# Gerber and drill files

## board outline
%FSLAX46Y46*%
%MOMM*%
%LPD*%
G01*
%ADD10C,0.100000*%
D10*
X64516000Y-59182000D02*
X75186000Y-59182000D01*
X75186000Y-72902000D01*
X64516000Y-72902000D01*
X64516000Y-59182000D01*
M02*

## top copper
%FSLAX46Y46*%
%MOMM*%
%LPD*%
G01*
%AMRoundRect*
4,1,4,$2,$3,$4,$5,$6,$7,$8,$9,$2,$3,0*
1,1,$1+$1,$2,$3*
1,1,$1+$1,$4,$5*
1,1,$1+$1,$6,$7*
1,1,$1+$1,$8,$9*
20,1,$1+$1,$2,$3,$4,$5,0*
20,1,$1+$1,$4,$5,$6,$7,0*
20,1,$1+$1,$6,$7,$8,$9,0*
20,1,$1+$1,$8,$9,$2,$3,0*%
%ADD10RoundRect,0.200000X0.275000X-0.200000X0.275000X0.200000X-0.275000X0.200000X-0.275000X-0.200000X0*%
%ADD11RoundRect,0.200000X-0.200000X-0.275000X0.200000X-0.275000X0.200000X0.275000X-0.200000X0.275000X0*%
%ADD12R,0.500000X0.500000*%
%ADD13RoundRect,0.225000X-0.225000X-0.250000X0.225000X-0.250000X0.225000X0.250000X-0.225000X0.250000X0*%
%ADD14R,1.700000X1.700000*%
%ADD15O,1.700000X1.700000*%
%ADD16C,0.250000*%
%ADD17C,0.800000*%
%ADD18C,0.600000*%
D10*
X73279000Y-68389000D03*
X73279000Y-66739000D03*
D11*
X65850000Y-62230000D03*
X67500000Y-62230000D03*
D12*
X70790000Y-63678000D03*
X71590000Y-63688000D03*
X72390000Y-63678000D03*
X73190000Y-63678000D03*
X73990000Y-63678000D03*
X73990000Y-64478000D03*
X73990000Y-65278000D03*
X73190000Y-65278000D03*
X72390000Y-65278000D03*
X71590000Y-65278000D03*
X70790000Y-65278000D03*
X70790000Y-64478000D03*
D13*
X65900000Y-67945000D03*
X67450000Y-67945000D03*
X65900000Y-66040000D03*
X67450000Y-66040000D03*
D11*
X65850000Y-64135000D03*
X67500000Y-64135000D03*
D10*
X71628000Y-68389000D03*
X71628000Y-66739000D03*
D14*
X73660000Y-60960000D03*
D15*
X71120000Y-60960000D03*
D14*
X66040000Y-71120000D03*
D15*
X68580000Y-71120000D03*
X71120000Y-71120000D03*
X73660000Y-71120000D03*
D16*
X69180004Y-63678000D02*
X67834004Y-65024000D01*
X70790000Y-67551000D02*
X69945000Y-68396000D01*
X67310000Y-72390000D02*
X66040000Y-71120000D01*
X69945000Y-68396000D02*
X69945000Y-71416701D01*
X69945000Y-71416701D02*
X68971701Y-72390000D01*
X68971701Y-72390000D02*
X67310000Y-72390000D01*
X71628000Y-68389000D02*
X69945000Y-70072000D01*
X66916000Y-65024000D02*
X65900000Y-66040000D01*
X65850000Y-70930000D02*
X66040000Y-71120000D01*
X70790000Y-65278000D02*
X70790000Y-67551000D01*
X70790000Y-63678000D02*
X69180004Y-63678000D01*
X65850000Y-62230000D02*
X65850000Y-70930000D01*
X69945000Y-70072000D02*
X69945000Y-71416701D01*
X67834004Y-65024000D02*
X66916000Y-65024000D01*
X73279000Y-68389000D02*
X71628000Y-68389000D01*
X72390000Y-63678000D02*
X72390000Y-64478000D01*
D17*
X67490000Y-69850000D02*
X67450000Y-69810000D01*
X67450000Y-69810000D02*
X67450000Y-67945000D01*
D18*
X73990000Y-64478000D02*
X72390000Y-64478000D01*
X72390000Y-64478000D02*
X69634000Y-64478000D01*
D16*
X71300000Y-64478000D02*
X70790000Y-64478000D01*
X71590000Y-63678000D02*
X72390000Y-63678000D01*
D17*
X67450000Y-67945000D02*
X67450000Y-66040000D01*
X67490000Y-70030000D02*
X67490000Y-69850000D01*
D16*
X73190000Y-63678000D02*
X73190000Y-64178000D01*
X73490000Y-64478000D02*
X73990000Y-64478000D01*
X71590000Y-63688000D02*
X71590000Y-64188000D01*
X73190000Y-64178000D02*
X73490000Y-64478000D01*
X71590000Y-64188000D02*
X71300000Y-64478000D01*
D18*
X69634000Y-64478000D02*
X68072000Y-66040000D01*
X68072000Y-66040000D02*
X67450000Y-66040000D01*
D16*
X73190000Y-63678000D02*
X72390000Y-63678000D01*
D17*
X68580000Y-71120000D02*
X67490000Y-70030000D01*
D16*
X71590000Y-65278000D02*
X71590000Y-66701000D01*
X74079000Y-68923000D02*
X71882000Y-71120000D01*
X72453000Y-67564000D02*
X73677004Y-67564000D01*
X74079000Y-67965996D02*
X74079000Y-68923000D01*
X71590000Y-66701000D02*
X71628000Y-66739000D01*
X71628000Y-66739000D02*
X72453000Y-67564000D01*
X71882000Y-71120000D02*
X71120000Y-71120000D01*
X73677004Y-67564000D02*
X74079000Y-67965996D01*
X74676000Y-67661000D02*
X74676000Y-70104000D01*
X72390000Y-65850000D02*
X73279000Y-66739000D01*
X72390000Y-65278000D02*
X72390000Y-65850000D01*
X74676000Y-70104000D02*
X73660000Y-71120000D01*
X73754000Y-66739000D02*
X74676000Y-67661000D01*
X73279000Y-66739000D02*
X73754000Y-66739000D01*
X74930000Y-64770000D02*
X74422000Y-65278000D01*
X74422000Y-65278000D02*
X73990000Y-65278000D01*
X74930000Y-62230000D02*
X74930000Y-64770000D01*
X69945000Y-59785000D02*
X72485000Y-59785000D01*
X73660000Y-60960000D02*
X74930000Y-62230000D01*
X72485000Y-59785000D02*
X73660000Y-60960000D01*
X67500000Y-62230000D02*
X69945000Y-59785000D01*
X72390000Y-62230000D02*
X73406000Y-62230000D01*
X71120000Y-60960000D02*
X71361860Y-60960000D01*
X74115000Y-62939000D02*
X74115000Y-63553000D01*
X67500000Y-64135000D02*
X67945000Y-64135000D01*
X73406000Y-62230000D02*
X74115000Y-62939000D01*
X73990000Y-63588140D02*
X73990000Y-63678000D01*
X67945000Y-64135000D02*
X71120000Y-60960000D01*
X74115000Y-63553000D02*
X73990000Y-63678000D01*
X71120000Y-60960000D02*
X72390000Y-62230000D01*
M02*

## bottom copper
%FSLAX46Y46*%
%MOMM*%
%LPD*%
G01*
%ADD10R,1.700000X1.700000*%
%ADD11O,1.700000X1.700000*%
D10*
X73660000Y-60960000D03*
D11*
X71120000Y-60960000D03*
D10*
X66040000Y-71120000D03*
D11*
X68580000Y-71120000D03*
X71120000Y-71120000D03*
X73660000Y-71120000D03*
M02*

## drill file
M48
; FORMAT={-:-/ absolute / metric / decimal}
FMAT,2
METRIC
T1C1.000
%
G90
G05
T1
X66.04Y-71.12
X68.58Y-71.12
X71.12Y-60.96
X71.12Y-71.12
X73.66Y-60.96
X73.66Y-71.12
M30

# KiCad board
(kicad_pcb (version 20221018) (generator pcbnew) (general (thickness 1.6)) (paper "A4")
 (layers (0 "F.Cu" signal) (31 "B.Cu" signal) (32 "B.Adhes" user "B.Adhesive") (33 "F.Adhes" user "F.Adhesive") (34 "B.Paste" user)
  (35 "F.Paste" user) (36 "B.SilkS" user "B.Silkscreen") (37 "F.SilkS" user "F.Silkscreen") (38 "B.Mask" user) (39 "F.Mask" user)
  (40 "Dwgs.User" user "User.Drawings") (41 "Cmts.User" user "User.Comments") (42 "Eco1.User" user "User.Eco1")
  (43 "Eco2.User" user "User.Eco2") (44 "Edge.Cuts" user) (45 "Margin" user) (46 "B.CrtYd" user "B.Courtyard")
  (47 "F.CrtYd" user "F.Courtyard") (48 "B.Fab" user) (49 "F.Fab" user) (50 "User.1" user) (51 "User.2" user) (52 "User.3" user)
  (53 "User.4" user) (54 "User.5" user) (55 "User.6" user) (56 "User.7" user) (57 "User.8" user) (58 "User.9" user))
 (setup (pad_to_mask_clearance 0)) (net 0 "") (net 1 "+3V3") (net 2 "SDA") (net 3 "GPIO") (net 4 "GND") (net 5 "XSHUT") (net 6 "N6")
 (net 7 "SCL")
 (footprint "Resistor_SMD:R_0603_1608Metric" (layer "F.Cu") (at 73.279 67.564 90)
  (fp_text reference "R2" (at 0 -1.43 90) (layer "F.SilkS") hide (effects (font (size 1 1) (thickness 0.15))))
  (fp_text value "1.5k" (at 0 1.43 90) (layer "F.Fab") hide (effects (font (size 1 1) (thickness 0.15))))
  (pad "1" smd roundrect (at -0.825 0 90) (size 0.8 0.95) (layers "F.Cu" "F.Paste" "F.Mask") (roundrect_rratio 0.25) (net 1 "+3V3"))
  (pad "2" smd roundrect (at 0.825 0 90) (size 0.8 0.95) (layers "F.Cu" "F.Paste" "F.Mask") (roundrect_rratio 0.25) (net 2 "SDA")))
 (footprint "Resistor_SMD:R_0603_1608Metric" (layer "F.Cu") (at 66.675 62.23)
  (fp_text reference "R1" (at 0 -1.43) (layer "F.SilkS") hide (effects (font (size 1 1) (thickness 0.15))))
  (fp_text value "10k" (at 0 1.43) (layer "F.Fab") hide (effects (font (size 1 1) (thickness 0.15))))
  (pad "1" smd roundrect (at -0.825 0) (size 0.8 0.95) (layers "F.Cu" "F.Paste" "F.Mask") (roundrect_rratio 0.25) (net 1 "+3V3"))
  (pad "2" smd roundrect (at 0.825 0) (size 0.8 0.95) (layers "F.Cu" "F.Paste" "F.Mask") (roundrect_rratio 0.25) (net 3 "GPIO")))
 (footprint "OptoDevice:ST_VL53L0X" (layer "F.Cu") (at 72.39 64.478)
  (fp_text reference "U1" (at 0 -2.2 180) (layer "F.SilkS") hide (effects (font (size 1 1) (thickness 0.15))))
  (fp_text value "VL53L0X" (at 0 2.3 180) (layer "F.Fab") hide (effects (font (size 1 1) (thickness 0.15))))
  (pad "1" smd rect (at -1.6 -0.8 90) (size 0.5 0.5) (layers "F.Cu" "F.Paste" "F.Mask") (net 1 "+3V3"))
  (pad "2" smd rect (at -0.8 -0.79 90) (size 0.5 0.5) (layers "F.Cu" "F.Paste" "F.Mask") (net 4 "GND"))
  (pad "3" smd rect (at 0 -0.8 90) (size 0.5 0.5) (layers "F.Cu" "F.Paste" "F.Mask") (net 4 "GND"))
  (pad "4" smd rect (at 0.8 -0.8 90) (size 0.5 0.5) (layers "F.Cu" "F.Paste" "F.Mask") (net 4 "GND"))
  (pad "5" smd rect (at 1.6 -0.8 90) (size 0.5 0.5) (layers "F.Cu" "F.Paste" "F.Mask") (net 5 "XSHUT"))
  (pad "6" smd rect (at 1.6 0 90) (size 0.5 0.5) (layers "F.Cu" "F.Paste" "F.Mask") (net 4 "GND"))
  (pad "7" smd rect (at 1.6 0.8 90) (size 0.5 0.5) (layers "F.Cu" "F.Paste" "F.Mask") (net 3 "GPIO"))
  (pad "8" smd rect (at 0.8 0.8 90) (size 0.5 0.5) (layers "F.Cu" "F.Paste" "F.Mask") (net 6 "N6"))
  (pad "9" smd rect (at 0 0.8 90) (size 0.5 0.5) (layers "F.Cu" "F.Paste" "F.Mask") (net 2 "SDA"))
  (pad "10" smd rect (at -0.8 0.8 90) (size 0.5 0.5) (layers "F.Cu" "F.Paste" "F.Mask") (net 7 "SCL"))
  (pad "11" smd rect (at -1.6 0.8 90) (size 0.5 0.5) (layers "F.Cu" "F.Paste" "F.Mask") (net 1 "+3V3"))
  (pad "12" smd rect (at -1.6 0 90) (size 0.5 0.5) (layers "F.Cu" "F.Paste" "F.Mask") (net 4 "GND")))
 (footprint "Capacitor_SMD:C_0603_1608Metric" (layer "F.Cu") (at 66.675 67.945)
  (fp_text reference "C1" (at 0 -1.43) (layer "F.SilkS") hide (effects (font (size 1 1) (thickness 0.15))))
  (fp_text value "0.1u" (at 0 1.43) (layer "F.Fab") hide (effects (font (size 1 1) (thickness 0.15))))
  (pad "1" smd roundrect (at -0.775 0) (size 0.9 0.95) (layers "F.Cu" "F.Paste" "F.Mask") (roundrect_rratio 0.25) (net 1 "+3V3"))
  (pad "2" smd roundrect (at 0.775 0) (size 0.9 0.95) (layers "F.Cu" "F.Paste" "F.Mask") (roundrect_rratio 0.25) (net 4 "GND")))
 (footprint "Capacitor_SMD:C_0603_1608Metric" (layer "F.Cu") (at 66.675 66.04)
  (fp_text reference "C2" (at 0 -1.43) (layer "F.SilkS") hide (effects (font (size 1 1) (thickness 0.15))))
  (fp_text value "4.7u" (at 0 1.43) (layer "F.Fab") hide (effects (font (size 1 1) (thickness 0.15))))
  (pad "1" smd roundrect (at -0.775 0) (size 0.9 0.95) (layers "F.Cu" "F.Paste" "F.Mask") (roundrect_rratio 0.25) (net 1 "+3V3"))
  (pad "2" smd roundrect (at 0.775 0) (size 0.9 0.95) (layers "F.Cu" "F.Paste" "F.Mask") (roundrect_rratio 0.25) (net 4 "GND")))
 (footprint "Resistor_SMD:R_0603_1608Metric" (layer "F.Cu") (at 66.675 64.135)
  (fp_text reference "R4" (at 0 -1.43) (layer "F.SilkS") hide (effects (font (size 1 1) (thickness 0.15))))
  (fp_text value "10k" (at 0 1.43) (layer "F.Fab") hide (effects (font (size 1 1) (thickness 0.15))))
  (pad "1" smd roundrect (at -0.825 0) (size 0.8 0.95) (layers "F.Cu" "F.Paste" "F.Mask") (roundrect_rratio 0.25) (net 1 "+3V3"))
  (pad "2" smd roundrect (at 0.825 0) (size 0.8 0.95) (layers "F.Cu" "F.Paste" "F.Mask") (roundrect_rratio 0.25) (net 5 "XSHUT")))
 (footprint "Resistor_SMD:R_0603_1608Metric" (layer "F.Cu") (at 71.628 67.564 90)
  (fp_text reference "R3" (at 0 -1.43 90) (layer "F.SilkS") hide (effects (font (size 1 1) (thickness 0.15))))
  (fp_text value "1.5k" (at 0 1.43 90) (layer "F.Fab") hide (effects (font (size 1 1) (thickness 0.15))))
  (pad "1" smd roundrect (at -0.825 0 90) (size 0.8 0.95) (layers "F.Cu" "F.Paste" "F.Mask") (roundrect_rratio 0.25) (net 1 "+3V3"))
  (pad "2" smd roundrect (at 0.825 0 90) (size 0.8 0.95) (layers "F.Cu" "F.Paste" "F.Mask") (roundrect_rratio 0.25) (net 7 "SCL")))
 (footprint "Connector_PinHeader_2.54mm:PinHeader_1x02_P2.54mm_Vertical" (layer "B.Cu") (at 73.66 60.96 90)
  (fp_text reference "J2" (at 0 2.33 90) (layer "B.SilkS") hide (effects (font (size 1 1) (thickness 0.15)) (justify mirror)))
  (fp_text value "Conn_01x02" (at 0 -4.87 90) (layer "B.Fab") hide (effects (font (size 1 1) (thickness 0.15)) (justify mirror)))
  (pad "1" thru_hole rect (at 0 0 90) (size 1.7 1.7) (drill 1) (layers "*.Cu" "*.Mask") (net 3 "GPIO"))
  (pad "2" thru_hole oval (at 0 -2.54 90) (size 1.7 1.7) (drill 1) (layers "*.Cu" "*.Mask") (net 5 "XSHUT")))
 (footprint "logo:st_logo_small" (layer "B.Cu") (at 72.39 67.056 180)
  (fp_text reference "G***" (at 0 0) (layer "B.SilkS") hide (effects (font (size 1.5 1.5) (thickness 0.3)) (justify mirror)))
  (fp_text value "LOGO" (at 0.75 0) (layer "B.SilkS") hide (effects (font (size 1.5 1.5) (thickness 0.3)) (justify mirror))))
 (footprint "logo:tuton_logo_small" (layer "B.Cu") (at 67.056 66.802 180)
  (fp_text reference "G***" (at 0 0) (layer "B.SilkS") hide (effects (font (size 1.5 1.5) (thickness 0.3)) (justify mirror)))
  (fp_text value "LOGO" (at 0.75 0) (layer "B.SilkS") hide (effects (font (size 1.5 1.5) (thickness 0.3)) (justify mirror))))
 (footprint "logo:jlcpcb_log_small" (layer "B.Cu") (at 70.866 64.008 180)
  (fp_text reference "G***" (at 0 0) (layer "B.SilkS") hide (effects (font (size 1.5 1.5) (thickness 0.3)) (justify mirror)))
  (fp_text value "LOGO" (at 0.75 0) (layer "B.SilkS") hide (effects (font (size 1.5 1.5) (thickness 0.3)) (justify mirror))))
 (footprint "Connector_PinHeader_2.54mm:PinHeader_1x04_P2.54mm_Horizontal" (layer "B.Cu") (at 66.04 71.12 -90)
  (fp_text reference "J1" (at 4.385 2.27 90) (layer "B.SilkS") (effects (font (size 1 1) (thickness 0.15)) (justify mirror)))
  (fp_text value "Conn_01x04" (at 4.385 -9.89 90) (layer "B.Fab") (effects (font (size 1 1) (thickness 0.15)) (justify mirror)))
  (pad "1" thru_hole rect (at 0 0 270) (size 1.7 1.7) (drill 1) (layers "*.Cu" "*.Mask") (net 1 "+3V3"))
  (pad "2" thru_hole oval (at 0 -2.54 270) (size 1.7 1.7) (drill 1) (layers "*.Cu" "*.Mask") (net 4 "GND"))
  (pad "3" thru_hole oval (at 0 -5.08 270) (size 1.7 1.7) (drill 1) (layers "*.Cu" "*.Mask") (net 7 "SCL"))
  (pad "4" thru_hole oval (at 0 -7.62 270) (size 1.7 1.7) (drill 1) (layers "*.Cu" "*.Mask") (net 2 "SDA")))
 (gr_rect (start 64.516 59.182) (end 75.186 72.902) (stroke (width 0.1) (type default)) (fill none) (layer "Edge.Cuts"))
 (segment (start 69.180004 63.678) (end 67.834004 65.024) (width 0.25) (layer "F.Cu") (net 1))
 (segment (start 70.79 67.551) (end 69.945 68.396) (width 0.25) (layer "F.Cu") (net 1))
 (segment (start 67.31 72.39) (end 66.04 71.12) (width 0.25) (layer "F.Cu") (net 1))
 (segment (start 69.945 68.396) (end 69.945 71.416701) (width 0.25) (layer "F.Cu") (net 1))
 (segment (start 69.945 71.416701) (end 68.971701 72.39) (width 0.25) (layer "F.Cu") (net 1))
 (segment (start 68.971701 72.39) (end 67.31 72.39) (width 0.25) (layer "F.Cu") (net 1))
 (segment (start 71.628 68.389) (end 69.945 70.072) (width 0.25) (layer "F.Cu") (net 1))
 (segment (start 66.916 65.024) (end 65.9 66.04) (width 0.25) (layer "F.Cu") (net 1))
 (segment (start 65.85 70.93) (end 66.04 71.12) (width 0.25) (layer "F.Cu") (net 1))
 (segment (start 70.79 65.278) (end 70.79 67.551) (width 0.25) (layer "F.Cu") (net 1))
 (segment (start 70.79 63.678) (end 69.180004 63.678) (width 0.25) (layer "F.Cu") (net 1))
 (segment (start 65.85 62.23) (end 65.85 70.93) (width 0.25) (layer "F.Cu") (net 1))
 (segment (start 69.945 70.072) (end 69.945 71.416701) (width 0.25) (layer "F.Cu") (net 1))
 (segment (start 67.834004 65.024) (end 66.916 65.024) (width 0.25) (layer "F.Cu") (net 1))
 (segment (start 73.279 68.389) (end 71.628 68.389) (width 0.25) (layer "F.Cu") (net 1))
 (segment (start 72.39 63.678) (end 72.39 64.478) (width 0.25) (layer "F.Cu") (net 4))
 (segment (start 67.49 69.85) (end 67.45 69.81) (width 0.8) (layer "F.Cu") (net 4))
 (segment (start 67.45 69.81) (end 67.45 67.945) (width 0.8) (layer "F.Cu") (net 4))
 (segment (start 73.99 64.478) (end 72.39 64.478) (width 0.6) (layer "F.Cu") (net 4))
 (segment (start 72.39 64.478) (end 69.634 64.478) (width 0.6) (layer "F.Cu") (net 4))
 (segment (start 71.3 64.478) (end 70.79 64.478) (width 0.25) (layer "F.Cu") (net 4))
 (segment (start 71.59 63.678) (end 72.39 63.678) (width 0.25) (layer "F.Cu") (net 4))
 (segment (start 67.45 67.945) (end 67.45 66.04) (width 0.8) (layer "F.Cu") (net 4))
 (segment (start 67.49 70.03) (end 67.49 69.85) (width 0.8) (layer "F.Cu") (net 4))
 (segment (start 73.19 63.678) (end 73.19 64.178) (width 0.25) (layer "F.Cu") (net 4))
 (segment (start 73.49 64.478) (end 73.99 64.478) (width 0.25) (layer "F.Cu") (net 4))
 (segment (start 71.59 63.688) (end 71.59 64.188) (width 0.25) (layer "F.Cu") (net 4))
 (segment (start 73.19 64.178) (end 73.49 64.478) (width 0.25) (layer "F.Cu") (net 4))
 (segment (start 71.59 64.188) (end 71.3 64.478) (width 0.25) (layer "F.Cu") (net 4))
 (segment (start 69.634 64.478) (end 68.072 66.04) (width 0.6) (layer "F.Cu") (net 4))
 (segment (start 68.072 66.04) (end 67.45 66.04) (width 0.6) (layer "F.Cu") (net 4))
 (segment (start 73.19 63.678) (end 72.39 63.678) (width 0.25) (layer "F.Cu") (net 4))
 (segment (start 68.58 71.12) (end 67.49 70.03) (width 0.8) (layer "F.Cu") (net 4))
 (segment (start 71.59 65.278) (end 71.59 66.701) (width 0.25) (layer "F.Cu") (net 7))
 (segment (start 74.079 68.923) (end 71.882 71.12) (width 0.25) (layer "F.Cu") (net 7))
 (segment (start 72.453 67.564) (end 73.677004 67.564) (width 0.25) (layer "F.Cu") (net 7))
 (segment (start 74.079 67.965996) (end 74.079 68.923) (width 0.25) (layer "F.Cu") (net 7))
 (segment (start 71.59 66.701) (end 71.628 66.739) (width 0.25) (layer "F.Cu") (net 7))
 (segment (start 71.628 66.739) (end 72.453 67.564) (width 0.25) (layer "F.Cu") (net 7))
 (segment (start 71.882 71.12) (end 71.12 71.12) (width 0.25) (layer "F.Cu") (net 7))
 (segment (start 73.677004 67.564) (end 74.079 67.965996) (width 0.25) (layer "F.Cu") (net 7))
 (segment (start 74.676 67.661) (end 74.676 70.104) (width 0.25) (layer "F.Cu") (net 2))
 (segment (start 72.39 65.85) (end 73.279 66.739) (width 0.25) (layer "F.Cu") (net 2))
 (segment (start 72.39 65.278) (end 72.39 65.85) (width 0.25) (layer "F.Cu") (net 2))
 (segment (start 74.676 70.104) (end 73.66 71.12) (width 0.25) (layer "F.Cu") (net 2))
 (segment (start 73.754 66.739) (end 74.676 67.661) (width 0.25) (layer "F.Cu") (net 2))
 (segment (start 73.279 66.739) (end 73.754 66.739) (width 0.25) (layer "F.Cu") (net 2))
 (segment (start 74.93 64.77) (end 74.422 65.278) (width 0.25) (layer "F.Cu") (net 3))
 (segment (start 74.422 65.278) (end 73.99 65.278) (width 0.25) (layer "F.Cu") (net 3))
 (segment (start 74.93 62.23) (end 74.93 64.77) (width 0.25) (layer "F.Cu") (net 3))
 (segment (start 69.945 59.785) (end 72.485 59.785) (width 0.25) (layer "F.Cu") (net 3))
 (segment (start 73.66 60.96) (end 74.93 62.23) (width 0.25) (layer "F.Cu") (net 3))
 (segment (start 72.485 59.785) (end 73.66 60.96) (width 0.25) (layer "F.Cu") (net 3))
 (segment (start 67.5 62.23) (end 69.945 59.785) (width 0.25) (layer "F.Cu") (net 3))
 (segment (start 72.39 62.23) (end 73.406 62.23) (width 0.25) (layer "F.Cu") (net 5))
 (segment (start 71.12 60.96) (end 71.36186 60.96) (width 0.25) (layer "F.Cu") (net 5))
 (segment (start 74.115 62.939) (end 74.115 63.553) (width 0.25) (layer "F.Cu") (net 5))
 (segment (start 67.5 64.135) (end 67.945 64.135) (width 0.25) (layer "F.Cu") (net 5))
 (segment (start 73.406 62.23) (end 74.115 62.939) (width 0.25) (layer "F.Cu") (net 5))
 (segment (start 73.99 63.58814) (end 73.99 63.678) (width 0.25) (layer "F.Cu") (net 5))
 (segment (start 67.945 64.135) (end 71.12 60.96) (width 0.25) (layer "F.Cu") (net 5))
 (segment (start 74.115 63.553) (end 73.99 63.678) (width 0.25) (layer "F.Cu") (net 5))
 (segment (start 71.12 60.96) (end 72.39 62.23) (width 0.25) (layer "F.Cu") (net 5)))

